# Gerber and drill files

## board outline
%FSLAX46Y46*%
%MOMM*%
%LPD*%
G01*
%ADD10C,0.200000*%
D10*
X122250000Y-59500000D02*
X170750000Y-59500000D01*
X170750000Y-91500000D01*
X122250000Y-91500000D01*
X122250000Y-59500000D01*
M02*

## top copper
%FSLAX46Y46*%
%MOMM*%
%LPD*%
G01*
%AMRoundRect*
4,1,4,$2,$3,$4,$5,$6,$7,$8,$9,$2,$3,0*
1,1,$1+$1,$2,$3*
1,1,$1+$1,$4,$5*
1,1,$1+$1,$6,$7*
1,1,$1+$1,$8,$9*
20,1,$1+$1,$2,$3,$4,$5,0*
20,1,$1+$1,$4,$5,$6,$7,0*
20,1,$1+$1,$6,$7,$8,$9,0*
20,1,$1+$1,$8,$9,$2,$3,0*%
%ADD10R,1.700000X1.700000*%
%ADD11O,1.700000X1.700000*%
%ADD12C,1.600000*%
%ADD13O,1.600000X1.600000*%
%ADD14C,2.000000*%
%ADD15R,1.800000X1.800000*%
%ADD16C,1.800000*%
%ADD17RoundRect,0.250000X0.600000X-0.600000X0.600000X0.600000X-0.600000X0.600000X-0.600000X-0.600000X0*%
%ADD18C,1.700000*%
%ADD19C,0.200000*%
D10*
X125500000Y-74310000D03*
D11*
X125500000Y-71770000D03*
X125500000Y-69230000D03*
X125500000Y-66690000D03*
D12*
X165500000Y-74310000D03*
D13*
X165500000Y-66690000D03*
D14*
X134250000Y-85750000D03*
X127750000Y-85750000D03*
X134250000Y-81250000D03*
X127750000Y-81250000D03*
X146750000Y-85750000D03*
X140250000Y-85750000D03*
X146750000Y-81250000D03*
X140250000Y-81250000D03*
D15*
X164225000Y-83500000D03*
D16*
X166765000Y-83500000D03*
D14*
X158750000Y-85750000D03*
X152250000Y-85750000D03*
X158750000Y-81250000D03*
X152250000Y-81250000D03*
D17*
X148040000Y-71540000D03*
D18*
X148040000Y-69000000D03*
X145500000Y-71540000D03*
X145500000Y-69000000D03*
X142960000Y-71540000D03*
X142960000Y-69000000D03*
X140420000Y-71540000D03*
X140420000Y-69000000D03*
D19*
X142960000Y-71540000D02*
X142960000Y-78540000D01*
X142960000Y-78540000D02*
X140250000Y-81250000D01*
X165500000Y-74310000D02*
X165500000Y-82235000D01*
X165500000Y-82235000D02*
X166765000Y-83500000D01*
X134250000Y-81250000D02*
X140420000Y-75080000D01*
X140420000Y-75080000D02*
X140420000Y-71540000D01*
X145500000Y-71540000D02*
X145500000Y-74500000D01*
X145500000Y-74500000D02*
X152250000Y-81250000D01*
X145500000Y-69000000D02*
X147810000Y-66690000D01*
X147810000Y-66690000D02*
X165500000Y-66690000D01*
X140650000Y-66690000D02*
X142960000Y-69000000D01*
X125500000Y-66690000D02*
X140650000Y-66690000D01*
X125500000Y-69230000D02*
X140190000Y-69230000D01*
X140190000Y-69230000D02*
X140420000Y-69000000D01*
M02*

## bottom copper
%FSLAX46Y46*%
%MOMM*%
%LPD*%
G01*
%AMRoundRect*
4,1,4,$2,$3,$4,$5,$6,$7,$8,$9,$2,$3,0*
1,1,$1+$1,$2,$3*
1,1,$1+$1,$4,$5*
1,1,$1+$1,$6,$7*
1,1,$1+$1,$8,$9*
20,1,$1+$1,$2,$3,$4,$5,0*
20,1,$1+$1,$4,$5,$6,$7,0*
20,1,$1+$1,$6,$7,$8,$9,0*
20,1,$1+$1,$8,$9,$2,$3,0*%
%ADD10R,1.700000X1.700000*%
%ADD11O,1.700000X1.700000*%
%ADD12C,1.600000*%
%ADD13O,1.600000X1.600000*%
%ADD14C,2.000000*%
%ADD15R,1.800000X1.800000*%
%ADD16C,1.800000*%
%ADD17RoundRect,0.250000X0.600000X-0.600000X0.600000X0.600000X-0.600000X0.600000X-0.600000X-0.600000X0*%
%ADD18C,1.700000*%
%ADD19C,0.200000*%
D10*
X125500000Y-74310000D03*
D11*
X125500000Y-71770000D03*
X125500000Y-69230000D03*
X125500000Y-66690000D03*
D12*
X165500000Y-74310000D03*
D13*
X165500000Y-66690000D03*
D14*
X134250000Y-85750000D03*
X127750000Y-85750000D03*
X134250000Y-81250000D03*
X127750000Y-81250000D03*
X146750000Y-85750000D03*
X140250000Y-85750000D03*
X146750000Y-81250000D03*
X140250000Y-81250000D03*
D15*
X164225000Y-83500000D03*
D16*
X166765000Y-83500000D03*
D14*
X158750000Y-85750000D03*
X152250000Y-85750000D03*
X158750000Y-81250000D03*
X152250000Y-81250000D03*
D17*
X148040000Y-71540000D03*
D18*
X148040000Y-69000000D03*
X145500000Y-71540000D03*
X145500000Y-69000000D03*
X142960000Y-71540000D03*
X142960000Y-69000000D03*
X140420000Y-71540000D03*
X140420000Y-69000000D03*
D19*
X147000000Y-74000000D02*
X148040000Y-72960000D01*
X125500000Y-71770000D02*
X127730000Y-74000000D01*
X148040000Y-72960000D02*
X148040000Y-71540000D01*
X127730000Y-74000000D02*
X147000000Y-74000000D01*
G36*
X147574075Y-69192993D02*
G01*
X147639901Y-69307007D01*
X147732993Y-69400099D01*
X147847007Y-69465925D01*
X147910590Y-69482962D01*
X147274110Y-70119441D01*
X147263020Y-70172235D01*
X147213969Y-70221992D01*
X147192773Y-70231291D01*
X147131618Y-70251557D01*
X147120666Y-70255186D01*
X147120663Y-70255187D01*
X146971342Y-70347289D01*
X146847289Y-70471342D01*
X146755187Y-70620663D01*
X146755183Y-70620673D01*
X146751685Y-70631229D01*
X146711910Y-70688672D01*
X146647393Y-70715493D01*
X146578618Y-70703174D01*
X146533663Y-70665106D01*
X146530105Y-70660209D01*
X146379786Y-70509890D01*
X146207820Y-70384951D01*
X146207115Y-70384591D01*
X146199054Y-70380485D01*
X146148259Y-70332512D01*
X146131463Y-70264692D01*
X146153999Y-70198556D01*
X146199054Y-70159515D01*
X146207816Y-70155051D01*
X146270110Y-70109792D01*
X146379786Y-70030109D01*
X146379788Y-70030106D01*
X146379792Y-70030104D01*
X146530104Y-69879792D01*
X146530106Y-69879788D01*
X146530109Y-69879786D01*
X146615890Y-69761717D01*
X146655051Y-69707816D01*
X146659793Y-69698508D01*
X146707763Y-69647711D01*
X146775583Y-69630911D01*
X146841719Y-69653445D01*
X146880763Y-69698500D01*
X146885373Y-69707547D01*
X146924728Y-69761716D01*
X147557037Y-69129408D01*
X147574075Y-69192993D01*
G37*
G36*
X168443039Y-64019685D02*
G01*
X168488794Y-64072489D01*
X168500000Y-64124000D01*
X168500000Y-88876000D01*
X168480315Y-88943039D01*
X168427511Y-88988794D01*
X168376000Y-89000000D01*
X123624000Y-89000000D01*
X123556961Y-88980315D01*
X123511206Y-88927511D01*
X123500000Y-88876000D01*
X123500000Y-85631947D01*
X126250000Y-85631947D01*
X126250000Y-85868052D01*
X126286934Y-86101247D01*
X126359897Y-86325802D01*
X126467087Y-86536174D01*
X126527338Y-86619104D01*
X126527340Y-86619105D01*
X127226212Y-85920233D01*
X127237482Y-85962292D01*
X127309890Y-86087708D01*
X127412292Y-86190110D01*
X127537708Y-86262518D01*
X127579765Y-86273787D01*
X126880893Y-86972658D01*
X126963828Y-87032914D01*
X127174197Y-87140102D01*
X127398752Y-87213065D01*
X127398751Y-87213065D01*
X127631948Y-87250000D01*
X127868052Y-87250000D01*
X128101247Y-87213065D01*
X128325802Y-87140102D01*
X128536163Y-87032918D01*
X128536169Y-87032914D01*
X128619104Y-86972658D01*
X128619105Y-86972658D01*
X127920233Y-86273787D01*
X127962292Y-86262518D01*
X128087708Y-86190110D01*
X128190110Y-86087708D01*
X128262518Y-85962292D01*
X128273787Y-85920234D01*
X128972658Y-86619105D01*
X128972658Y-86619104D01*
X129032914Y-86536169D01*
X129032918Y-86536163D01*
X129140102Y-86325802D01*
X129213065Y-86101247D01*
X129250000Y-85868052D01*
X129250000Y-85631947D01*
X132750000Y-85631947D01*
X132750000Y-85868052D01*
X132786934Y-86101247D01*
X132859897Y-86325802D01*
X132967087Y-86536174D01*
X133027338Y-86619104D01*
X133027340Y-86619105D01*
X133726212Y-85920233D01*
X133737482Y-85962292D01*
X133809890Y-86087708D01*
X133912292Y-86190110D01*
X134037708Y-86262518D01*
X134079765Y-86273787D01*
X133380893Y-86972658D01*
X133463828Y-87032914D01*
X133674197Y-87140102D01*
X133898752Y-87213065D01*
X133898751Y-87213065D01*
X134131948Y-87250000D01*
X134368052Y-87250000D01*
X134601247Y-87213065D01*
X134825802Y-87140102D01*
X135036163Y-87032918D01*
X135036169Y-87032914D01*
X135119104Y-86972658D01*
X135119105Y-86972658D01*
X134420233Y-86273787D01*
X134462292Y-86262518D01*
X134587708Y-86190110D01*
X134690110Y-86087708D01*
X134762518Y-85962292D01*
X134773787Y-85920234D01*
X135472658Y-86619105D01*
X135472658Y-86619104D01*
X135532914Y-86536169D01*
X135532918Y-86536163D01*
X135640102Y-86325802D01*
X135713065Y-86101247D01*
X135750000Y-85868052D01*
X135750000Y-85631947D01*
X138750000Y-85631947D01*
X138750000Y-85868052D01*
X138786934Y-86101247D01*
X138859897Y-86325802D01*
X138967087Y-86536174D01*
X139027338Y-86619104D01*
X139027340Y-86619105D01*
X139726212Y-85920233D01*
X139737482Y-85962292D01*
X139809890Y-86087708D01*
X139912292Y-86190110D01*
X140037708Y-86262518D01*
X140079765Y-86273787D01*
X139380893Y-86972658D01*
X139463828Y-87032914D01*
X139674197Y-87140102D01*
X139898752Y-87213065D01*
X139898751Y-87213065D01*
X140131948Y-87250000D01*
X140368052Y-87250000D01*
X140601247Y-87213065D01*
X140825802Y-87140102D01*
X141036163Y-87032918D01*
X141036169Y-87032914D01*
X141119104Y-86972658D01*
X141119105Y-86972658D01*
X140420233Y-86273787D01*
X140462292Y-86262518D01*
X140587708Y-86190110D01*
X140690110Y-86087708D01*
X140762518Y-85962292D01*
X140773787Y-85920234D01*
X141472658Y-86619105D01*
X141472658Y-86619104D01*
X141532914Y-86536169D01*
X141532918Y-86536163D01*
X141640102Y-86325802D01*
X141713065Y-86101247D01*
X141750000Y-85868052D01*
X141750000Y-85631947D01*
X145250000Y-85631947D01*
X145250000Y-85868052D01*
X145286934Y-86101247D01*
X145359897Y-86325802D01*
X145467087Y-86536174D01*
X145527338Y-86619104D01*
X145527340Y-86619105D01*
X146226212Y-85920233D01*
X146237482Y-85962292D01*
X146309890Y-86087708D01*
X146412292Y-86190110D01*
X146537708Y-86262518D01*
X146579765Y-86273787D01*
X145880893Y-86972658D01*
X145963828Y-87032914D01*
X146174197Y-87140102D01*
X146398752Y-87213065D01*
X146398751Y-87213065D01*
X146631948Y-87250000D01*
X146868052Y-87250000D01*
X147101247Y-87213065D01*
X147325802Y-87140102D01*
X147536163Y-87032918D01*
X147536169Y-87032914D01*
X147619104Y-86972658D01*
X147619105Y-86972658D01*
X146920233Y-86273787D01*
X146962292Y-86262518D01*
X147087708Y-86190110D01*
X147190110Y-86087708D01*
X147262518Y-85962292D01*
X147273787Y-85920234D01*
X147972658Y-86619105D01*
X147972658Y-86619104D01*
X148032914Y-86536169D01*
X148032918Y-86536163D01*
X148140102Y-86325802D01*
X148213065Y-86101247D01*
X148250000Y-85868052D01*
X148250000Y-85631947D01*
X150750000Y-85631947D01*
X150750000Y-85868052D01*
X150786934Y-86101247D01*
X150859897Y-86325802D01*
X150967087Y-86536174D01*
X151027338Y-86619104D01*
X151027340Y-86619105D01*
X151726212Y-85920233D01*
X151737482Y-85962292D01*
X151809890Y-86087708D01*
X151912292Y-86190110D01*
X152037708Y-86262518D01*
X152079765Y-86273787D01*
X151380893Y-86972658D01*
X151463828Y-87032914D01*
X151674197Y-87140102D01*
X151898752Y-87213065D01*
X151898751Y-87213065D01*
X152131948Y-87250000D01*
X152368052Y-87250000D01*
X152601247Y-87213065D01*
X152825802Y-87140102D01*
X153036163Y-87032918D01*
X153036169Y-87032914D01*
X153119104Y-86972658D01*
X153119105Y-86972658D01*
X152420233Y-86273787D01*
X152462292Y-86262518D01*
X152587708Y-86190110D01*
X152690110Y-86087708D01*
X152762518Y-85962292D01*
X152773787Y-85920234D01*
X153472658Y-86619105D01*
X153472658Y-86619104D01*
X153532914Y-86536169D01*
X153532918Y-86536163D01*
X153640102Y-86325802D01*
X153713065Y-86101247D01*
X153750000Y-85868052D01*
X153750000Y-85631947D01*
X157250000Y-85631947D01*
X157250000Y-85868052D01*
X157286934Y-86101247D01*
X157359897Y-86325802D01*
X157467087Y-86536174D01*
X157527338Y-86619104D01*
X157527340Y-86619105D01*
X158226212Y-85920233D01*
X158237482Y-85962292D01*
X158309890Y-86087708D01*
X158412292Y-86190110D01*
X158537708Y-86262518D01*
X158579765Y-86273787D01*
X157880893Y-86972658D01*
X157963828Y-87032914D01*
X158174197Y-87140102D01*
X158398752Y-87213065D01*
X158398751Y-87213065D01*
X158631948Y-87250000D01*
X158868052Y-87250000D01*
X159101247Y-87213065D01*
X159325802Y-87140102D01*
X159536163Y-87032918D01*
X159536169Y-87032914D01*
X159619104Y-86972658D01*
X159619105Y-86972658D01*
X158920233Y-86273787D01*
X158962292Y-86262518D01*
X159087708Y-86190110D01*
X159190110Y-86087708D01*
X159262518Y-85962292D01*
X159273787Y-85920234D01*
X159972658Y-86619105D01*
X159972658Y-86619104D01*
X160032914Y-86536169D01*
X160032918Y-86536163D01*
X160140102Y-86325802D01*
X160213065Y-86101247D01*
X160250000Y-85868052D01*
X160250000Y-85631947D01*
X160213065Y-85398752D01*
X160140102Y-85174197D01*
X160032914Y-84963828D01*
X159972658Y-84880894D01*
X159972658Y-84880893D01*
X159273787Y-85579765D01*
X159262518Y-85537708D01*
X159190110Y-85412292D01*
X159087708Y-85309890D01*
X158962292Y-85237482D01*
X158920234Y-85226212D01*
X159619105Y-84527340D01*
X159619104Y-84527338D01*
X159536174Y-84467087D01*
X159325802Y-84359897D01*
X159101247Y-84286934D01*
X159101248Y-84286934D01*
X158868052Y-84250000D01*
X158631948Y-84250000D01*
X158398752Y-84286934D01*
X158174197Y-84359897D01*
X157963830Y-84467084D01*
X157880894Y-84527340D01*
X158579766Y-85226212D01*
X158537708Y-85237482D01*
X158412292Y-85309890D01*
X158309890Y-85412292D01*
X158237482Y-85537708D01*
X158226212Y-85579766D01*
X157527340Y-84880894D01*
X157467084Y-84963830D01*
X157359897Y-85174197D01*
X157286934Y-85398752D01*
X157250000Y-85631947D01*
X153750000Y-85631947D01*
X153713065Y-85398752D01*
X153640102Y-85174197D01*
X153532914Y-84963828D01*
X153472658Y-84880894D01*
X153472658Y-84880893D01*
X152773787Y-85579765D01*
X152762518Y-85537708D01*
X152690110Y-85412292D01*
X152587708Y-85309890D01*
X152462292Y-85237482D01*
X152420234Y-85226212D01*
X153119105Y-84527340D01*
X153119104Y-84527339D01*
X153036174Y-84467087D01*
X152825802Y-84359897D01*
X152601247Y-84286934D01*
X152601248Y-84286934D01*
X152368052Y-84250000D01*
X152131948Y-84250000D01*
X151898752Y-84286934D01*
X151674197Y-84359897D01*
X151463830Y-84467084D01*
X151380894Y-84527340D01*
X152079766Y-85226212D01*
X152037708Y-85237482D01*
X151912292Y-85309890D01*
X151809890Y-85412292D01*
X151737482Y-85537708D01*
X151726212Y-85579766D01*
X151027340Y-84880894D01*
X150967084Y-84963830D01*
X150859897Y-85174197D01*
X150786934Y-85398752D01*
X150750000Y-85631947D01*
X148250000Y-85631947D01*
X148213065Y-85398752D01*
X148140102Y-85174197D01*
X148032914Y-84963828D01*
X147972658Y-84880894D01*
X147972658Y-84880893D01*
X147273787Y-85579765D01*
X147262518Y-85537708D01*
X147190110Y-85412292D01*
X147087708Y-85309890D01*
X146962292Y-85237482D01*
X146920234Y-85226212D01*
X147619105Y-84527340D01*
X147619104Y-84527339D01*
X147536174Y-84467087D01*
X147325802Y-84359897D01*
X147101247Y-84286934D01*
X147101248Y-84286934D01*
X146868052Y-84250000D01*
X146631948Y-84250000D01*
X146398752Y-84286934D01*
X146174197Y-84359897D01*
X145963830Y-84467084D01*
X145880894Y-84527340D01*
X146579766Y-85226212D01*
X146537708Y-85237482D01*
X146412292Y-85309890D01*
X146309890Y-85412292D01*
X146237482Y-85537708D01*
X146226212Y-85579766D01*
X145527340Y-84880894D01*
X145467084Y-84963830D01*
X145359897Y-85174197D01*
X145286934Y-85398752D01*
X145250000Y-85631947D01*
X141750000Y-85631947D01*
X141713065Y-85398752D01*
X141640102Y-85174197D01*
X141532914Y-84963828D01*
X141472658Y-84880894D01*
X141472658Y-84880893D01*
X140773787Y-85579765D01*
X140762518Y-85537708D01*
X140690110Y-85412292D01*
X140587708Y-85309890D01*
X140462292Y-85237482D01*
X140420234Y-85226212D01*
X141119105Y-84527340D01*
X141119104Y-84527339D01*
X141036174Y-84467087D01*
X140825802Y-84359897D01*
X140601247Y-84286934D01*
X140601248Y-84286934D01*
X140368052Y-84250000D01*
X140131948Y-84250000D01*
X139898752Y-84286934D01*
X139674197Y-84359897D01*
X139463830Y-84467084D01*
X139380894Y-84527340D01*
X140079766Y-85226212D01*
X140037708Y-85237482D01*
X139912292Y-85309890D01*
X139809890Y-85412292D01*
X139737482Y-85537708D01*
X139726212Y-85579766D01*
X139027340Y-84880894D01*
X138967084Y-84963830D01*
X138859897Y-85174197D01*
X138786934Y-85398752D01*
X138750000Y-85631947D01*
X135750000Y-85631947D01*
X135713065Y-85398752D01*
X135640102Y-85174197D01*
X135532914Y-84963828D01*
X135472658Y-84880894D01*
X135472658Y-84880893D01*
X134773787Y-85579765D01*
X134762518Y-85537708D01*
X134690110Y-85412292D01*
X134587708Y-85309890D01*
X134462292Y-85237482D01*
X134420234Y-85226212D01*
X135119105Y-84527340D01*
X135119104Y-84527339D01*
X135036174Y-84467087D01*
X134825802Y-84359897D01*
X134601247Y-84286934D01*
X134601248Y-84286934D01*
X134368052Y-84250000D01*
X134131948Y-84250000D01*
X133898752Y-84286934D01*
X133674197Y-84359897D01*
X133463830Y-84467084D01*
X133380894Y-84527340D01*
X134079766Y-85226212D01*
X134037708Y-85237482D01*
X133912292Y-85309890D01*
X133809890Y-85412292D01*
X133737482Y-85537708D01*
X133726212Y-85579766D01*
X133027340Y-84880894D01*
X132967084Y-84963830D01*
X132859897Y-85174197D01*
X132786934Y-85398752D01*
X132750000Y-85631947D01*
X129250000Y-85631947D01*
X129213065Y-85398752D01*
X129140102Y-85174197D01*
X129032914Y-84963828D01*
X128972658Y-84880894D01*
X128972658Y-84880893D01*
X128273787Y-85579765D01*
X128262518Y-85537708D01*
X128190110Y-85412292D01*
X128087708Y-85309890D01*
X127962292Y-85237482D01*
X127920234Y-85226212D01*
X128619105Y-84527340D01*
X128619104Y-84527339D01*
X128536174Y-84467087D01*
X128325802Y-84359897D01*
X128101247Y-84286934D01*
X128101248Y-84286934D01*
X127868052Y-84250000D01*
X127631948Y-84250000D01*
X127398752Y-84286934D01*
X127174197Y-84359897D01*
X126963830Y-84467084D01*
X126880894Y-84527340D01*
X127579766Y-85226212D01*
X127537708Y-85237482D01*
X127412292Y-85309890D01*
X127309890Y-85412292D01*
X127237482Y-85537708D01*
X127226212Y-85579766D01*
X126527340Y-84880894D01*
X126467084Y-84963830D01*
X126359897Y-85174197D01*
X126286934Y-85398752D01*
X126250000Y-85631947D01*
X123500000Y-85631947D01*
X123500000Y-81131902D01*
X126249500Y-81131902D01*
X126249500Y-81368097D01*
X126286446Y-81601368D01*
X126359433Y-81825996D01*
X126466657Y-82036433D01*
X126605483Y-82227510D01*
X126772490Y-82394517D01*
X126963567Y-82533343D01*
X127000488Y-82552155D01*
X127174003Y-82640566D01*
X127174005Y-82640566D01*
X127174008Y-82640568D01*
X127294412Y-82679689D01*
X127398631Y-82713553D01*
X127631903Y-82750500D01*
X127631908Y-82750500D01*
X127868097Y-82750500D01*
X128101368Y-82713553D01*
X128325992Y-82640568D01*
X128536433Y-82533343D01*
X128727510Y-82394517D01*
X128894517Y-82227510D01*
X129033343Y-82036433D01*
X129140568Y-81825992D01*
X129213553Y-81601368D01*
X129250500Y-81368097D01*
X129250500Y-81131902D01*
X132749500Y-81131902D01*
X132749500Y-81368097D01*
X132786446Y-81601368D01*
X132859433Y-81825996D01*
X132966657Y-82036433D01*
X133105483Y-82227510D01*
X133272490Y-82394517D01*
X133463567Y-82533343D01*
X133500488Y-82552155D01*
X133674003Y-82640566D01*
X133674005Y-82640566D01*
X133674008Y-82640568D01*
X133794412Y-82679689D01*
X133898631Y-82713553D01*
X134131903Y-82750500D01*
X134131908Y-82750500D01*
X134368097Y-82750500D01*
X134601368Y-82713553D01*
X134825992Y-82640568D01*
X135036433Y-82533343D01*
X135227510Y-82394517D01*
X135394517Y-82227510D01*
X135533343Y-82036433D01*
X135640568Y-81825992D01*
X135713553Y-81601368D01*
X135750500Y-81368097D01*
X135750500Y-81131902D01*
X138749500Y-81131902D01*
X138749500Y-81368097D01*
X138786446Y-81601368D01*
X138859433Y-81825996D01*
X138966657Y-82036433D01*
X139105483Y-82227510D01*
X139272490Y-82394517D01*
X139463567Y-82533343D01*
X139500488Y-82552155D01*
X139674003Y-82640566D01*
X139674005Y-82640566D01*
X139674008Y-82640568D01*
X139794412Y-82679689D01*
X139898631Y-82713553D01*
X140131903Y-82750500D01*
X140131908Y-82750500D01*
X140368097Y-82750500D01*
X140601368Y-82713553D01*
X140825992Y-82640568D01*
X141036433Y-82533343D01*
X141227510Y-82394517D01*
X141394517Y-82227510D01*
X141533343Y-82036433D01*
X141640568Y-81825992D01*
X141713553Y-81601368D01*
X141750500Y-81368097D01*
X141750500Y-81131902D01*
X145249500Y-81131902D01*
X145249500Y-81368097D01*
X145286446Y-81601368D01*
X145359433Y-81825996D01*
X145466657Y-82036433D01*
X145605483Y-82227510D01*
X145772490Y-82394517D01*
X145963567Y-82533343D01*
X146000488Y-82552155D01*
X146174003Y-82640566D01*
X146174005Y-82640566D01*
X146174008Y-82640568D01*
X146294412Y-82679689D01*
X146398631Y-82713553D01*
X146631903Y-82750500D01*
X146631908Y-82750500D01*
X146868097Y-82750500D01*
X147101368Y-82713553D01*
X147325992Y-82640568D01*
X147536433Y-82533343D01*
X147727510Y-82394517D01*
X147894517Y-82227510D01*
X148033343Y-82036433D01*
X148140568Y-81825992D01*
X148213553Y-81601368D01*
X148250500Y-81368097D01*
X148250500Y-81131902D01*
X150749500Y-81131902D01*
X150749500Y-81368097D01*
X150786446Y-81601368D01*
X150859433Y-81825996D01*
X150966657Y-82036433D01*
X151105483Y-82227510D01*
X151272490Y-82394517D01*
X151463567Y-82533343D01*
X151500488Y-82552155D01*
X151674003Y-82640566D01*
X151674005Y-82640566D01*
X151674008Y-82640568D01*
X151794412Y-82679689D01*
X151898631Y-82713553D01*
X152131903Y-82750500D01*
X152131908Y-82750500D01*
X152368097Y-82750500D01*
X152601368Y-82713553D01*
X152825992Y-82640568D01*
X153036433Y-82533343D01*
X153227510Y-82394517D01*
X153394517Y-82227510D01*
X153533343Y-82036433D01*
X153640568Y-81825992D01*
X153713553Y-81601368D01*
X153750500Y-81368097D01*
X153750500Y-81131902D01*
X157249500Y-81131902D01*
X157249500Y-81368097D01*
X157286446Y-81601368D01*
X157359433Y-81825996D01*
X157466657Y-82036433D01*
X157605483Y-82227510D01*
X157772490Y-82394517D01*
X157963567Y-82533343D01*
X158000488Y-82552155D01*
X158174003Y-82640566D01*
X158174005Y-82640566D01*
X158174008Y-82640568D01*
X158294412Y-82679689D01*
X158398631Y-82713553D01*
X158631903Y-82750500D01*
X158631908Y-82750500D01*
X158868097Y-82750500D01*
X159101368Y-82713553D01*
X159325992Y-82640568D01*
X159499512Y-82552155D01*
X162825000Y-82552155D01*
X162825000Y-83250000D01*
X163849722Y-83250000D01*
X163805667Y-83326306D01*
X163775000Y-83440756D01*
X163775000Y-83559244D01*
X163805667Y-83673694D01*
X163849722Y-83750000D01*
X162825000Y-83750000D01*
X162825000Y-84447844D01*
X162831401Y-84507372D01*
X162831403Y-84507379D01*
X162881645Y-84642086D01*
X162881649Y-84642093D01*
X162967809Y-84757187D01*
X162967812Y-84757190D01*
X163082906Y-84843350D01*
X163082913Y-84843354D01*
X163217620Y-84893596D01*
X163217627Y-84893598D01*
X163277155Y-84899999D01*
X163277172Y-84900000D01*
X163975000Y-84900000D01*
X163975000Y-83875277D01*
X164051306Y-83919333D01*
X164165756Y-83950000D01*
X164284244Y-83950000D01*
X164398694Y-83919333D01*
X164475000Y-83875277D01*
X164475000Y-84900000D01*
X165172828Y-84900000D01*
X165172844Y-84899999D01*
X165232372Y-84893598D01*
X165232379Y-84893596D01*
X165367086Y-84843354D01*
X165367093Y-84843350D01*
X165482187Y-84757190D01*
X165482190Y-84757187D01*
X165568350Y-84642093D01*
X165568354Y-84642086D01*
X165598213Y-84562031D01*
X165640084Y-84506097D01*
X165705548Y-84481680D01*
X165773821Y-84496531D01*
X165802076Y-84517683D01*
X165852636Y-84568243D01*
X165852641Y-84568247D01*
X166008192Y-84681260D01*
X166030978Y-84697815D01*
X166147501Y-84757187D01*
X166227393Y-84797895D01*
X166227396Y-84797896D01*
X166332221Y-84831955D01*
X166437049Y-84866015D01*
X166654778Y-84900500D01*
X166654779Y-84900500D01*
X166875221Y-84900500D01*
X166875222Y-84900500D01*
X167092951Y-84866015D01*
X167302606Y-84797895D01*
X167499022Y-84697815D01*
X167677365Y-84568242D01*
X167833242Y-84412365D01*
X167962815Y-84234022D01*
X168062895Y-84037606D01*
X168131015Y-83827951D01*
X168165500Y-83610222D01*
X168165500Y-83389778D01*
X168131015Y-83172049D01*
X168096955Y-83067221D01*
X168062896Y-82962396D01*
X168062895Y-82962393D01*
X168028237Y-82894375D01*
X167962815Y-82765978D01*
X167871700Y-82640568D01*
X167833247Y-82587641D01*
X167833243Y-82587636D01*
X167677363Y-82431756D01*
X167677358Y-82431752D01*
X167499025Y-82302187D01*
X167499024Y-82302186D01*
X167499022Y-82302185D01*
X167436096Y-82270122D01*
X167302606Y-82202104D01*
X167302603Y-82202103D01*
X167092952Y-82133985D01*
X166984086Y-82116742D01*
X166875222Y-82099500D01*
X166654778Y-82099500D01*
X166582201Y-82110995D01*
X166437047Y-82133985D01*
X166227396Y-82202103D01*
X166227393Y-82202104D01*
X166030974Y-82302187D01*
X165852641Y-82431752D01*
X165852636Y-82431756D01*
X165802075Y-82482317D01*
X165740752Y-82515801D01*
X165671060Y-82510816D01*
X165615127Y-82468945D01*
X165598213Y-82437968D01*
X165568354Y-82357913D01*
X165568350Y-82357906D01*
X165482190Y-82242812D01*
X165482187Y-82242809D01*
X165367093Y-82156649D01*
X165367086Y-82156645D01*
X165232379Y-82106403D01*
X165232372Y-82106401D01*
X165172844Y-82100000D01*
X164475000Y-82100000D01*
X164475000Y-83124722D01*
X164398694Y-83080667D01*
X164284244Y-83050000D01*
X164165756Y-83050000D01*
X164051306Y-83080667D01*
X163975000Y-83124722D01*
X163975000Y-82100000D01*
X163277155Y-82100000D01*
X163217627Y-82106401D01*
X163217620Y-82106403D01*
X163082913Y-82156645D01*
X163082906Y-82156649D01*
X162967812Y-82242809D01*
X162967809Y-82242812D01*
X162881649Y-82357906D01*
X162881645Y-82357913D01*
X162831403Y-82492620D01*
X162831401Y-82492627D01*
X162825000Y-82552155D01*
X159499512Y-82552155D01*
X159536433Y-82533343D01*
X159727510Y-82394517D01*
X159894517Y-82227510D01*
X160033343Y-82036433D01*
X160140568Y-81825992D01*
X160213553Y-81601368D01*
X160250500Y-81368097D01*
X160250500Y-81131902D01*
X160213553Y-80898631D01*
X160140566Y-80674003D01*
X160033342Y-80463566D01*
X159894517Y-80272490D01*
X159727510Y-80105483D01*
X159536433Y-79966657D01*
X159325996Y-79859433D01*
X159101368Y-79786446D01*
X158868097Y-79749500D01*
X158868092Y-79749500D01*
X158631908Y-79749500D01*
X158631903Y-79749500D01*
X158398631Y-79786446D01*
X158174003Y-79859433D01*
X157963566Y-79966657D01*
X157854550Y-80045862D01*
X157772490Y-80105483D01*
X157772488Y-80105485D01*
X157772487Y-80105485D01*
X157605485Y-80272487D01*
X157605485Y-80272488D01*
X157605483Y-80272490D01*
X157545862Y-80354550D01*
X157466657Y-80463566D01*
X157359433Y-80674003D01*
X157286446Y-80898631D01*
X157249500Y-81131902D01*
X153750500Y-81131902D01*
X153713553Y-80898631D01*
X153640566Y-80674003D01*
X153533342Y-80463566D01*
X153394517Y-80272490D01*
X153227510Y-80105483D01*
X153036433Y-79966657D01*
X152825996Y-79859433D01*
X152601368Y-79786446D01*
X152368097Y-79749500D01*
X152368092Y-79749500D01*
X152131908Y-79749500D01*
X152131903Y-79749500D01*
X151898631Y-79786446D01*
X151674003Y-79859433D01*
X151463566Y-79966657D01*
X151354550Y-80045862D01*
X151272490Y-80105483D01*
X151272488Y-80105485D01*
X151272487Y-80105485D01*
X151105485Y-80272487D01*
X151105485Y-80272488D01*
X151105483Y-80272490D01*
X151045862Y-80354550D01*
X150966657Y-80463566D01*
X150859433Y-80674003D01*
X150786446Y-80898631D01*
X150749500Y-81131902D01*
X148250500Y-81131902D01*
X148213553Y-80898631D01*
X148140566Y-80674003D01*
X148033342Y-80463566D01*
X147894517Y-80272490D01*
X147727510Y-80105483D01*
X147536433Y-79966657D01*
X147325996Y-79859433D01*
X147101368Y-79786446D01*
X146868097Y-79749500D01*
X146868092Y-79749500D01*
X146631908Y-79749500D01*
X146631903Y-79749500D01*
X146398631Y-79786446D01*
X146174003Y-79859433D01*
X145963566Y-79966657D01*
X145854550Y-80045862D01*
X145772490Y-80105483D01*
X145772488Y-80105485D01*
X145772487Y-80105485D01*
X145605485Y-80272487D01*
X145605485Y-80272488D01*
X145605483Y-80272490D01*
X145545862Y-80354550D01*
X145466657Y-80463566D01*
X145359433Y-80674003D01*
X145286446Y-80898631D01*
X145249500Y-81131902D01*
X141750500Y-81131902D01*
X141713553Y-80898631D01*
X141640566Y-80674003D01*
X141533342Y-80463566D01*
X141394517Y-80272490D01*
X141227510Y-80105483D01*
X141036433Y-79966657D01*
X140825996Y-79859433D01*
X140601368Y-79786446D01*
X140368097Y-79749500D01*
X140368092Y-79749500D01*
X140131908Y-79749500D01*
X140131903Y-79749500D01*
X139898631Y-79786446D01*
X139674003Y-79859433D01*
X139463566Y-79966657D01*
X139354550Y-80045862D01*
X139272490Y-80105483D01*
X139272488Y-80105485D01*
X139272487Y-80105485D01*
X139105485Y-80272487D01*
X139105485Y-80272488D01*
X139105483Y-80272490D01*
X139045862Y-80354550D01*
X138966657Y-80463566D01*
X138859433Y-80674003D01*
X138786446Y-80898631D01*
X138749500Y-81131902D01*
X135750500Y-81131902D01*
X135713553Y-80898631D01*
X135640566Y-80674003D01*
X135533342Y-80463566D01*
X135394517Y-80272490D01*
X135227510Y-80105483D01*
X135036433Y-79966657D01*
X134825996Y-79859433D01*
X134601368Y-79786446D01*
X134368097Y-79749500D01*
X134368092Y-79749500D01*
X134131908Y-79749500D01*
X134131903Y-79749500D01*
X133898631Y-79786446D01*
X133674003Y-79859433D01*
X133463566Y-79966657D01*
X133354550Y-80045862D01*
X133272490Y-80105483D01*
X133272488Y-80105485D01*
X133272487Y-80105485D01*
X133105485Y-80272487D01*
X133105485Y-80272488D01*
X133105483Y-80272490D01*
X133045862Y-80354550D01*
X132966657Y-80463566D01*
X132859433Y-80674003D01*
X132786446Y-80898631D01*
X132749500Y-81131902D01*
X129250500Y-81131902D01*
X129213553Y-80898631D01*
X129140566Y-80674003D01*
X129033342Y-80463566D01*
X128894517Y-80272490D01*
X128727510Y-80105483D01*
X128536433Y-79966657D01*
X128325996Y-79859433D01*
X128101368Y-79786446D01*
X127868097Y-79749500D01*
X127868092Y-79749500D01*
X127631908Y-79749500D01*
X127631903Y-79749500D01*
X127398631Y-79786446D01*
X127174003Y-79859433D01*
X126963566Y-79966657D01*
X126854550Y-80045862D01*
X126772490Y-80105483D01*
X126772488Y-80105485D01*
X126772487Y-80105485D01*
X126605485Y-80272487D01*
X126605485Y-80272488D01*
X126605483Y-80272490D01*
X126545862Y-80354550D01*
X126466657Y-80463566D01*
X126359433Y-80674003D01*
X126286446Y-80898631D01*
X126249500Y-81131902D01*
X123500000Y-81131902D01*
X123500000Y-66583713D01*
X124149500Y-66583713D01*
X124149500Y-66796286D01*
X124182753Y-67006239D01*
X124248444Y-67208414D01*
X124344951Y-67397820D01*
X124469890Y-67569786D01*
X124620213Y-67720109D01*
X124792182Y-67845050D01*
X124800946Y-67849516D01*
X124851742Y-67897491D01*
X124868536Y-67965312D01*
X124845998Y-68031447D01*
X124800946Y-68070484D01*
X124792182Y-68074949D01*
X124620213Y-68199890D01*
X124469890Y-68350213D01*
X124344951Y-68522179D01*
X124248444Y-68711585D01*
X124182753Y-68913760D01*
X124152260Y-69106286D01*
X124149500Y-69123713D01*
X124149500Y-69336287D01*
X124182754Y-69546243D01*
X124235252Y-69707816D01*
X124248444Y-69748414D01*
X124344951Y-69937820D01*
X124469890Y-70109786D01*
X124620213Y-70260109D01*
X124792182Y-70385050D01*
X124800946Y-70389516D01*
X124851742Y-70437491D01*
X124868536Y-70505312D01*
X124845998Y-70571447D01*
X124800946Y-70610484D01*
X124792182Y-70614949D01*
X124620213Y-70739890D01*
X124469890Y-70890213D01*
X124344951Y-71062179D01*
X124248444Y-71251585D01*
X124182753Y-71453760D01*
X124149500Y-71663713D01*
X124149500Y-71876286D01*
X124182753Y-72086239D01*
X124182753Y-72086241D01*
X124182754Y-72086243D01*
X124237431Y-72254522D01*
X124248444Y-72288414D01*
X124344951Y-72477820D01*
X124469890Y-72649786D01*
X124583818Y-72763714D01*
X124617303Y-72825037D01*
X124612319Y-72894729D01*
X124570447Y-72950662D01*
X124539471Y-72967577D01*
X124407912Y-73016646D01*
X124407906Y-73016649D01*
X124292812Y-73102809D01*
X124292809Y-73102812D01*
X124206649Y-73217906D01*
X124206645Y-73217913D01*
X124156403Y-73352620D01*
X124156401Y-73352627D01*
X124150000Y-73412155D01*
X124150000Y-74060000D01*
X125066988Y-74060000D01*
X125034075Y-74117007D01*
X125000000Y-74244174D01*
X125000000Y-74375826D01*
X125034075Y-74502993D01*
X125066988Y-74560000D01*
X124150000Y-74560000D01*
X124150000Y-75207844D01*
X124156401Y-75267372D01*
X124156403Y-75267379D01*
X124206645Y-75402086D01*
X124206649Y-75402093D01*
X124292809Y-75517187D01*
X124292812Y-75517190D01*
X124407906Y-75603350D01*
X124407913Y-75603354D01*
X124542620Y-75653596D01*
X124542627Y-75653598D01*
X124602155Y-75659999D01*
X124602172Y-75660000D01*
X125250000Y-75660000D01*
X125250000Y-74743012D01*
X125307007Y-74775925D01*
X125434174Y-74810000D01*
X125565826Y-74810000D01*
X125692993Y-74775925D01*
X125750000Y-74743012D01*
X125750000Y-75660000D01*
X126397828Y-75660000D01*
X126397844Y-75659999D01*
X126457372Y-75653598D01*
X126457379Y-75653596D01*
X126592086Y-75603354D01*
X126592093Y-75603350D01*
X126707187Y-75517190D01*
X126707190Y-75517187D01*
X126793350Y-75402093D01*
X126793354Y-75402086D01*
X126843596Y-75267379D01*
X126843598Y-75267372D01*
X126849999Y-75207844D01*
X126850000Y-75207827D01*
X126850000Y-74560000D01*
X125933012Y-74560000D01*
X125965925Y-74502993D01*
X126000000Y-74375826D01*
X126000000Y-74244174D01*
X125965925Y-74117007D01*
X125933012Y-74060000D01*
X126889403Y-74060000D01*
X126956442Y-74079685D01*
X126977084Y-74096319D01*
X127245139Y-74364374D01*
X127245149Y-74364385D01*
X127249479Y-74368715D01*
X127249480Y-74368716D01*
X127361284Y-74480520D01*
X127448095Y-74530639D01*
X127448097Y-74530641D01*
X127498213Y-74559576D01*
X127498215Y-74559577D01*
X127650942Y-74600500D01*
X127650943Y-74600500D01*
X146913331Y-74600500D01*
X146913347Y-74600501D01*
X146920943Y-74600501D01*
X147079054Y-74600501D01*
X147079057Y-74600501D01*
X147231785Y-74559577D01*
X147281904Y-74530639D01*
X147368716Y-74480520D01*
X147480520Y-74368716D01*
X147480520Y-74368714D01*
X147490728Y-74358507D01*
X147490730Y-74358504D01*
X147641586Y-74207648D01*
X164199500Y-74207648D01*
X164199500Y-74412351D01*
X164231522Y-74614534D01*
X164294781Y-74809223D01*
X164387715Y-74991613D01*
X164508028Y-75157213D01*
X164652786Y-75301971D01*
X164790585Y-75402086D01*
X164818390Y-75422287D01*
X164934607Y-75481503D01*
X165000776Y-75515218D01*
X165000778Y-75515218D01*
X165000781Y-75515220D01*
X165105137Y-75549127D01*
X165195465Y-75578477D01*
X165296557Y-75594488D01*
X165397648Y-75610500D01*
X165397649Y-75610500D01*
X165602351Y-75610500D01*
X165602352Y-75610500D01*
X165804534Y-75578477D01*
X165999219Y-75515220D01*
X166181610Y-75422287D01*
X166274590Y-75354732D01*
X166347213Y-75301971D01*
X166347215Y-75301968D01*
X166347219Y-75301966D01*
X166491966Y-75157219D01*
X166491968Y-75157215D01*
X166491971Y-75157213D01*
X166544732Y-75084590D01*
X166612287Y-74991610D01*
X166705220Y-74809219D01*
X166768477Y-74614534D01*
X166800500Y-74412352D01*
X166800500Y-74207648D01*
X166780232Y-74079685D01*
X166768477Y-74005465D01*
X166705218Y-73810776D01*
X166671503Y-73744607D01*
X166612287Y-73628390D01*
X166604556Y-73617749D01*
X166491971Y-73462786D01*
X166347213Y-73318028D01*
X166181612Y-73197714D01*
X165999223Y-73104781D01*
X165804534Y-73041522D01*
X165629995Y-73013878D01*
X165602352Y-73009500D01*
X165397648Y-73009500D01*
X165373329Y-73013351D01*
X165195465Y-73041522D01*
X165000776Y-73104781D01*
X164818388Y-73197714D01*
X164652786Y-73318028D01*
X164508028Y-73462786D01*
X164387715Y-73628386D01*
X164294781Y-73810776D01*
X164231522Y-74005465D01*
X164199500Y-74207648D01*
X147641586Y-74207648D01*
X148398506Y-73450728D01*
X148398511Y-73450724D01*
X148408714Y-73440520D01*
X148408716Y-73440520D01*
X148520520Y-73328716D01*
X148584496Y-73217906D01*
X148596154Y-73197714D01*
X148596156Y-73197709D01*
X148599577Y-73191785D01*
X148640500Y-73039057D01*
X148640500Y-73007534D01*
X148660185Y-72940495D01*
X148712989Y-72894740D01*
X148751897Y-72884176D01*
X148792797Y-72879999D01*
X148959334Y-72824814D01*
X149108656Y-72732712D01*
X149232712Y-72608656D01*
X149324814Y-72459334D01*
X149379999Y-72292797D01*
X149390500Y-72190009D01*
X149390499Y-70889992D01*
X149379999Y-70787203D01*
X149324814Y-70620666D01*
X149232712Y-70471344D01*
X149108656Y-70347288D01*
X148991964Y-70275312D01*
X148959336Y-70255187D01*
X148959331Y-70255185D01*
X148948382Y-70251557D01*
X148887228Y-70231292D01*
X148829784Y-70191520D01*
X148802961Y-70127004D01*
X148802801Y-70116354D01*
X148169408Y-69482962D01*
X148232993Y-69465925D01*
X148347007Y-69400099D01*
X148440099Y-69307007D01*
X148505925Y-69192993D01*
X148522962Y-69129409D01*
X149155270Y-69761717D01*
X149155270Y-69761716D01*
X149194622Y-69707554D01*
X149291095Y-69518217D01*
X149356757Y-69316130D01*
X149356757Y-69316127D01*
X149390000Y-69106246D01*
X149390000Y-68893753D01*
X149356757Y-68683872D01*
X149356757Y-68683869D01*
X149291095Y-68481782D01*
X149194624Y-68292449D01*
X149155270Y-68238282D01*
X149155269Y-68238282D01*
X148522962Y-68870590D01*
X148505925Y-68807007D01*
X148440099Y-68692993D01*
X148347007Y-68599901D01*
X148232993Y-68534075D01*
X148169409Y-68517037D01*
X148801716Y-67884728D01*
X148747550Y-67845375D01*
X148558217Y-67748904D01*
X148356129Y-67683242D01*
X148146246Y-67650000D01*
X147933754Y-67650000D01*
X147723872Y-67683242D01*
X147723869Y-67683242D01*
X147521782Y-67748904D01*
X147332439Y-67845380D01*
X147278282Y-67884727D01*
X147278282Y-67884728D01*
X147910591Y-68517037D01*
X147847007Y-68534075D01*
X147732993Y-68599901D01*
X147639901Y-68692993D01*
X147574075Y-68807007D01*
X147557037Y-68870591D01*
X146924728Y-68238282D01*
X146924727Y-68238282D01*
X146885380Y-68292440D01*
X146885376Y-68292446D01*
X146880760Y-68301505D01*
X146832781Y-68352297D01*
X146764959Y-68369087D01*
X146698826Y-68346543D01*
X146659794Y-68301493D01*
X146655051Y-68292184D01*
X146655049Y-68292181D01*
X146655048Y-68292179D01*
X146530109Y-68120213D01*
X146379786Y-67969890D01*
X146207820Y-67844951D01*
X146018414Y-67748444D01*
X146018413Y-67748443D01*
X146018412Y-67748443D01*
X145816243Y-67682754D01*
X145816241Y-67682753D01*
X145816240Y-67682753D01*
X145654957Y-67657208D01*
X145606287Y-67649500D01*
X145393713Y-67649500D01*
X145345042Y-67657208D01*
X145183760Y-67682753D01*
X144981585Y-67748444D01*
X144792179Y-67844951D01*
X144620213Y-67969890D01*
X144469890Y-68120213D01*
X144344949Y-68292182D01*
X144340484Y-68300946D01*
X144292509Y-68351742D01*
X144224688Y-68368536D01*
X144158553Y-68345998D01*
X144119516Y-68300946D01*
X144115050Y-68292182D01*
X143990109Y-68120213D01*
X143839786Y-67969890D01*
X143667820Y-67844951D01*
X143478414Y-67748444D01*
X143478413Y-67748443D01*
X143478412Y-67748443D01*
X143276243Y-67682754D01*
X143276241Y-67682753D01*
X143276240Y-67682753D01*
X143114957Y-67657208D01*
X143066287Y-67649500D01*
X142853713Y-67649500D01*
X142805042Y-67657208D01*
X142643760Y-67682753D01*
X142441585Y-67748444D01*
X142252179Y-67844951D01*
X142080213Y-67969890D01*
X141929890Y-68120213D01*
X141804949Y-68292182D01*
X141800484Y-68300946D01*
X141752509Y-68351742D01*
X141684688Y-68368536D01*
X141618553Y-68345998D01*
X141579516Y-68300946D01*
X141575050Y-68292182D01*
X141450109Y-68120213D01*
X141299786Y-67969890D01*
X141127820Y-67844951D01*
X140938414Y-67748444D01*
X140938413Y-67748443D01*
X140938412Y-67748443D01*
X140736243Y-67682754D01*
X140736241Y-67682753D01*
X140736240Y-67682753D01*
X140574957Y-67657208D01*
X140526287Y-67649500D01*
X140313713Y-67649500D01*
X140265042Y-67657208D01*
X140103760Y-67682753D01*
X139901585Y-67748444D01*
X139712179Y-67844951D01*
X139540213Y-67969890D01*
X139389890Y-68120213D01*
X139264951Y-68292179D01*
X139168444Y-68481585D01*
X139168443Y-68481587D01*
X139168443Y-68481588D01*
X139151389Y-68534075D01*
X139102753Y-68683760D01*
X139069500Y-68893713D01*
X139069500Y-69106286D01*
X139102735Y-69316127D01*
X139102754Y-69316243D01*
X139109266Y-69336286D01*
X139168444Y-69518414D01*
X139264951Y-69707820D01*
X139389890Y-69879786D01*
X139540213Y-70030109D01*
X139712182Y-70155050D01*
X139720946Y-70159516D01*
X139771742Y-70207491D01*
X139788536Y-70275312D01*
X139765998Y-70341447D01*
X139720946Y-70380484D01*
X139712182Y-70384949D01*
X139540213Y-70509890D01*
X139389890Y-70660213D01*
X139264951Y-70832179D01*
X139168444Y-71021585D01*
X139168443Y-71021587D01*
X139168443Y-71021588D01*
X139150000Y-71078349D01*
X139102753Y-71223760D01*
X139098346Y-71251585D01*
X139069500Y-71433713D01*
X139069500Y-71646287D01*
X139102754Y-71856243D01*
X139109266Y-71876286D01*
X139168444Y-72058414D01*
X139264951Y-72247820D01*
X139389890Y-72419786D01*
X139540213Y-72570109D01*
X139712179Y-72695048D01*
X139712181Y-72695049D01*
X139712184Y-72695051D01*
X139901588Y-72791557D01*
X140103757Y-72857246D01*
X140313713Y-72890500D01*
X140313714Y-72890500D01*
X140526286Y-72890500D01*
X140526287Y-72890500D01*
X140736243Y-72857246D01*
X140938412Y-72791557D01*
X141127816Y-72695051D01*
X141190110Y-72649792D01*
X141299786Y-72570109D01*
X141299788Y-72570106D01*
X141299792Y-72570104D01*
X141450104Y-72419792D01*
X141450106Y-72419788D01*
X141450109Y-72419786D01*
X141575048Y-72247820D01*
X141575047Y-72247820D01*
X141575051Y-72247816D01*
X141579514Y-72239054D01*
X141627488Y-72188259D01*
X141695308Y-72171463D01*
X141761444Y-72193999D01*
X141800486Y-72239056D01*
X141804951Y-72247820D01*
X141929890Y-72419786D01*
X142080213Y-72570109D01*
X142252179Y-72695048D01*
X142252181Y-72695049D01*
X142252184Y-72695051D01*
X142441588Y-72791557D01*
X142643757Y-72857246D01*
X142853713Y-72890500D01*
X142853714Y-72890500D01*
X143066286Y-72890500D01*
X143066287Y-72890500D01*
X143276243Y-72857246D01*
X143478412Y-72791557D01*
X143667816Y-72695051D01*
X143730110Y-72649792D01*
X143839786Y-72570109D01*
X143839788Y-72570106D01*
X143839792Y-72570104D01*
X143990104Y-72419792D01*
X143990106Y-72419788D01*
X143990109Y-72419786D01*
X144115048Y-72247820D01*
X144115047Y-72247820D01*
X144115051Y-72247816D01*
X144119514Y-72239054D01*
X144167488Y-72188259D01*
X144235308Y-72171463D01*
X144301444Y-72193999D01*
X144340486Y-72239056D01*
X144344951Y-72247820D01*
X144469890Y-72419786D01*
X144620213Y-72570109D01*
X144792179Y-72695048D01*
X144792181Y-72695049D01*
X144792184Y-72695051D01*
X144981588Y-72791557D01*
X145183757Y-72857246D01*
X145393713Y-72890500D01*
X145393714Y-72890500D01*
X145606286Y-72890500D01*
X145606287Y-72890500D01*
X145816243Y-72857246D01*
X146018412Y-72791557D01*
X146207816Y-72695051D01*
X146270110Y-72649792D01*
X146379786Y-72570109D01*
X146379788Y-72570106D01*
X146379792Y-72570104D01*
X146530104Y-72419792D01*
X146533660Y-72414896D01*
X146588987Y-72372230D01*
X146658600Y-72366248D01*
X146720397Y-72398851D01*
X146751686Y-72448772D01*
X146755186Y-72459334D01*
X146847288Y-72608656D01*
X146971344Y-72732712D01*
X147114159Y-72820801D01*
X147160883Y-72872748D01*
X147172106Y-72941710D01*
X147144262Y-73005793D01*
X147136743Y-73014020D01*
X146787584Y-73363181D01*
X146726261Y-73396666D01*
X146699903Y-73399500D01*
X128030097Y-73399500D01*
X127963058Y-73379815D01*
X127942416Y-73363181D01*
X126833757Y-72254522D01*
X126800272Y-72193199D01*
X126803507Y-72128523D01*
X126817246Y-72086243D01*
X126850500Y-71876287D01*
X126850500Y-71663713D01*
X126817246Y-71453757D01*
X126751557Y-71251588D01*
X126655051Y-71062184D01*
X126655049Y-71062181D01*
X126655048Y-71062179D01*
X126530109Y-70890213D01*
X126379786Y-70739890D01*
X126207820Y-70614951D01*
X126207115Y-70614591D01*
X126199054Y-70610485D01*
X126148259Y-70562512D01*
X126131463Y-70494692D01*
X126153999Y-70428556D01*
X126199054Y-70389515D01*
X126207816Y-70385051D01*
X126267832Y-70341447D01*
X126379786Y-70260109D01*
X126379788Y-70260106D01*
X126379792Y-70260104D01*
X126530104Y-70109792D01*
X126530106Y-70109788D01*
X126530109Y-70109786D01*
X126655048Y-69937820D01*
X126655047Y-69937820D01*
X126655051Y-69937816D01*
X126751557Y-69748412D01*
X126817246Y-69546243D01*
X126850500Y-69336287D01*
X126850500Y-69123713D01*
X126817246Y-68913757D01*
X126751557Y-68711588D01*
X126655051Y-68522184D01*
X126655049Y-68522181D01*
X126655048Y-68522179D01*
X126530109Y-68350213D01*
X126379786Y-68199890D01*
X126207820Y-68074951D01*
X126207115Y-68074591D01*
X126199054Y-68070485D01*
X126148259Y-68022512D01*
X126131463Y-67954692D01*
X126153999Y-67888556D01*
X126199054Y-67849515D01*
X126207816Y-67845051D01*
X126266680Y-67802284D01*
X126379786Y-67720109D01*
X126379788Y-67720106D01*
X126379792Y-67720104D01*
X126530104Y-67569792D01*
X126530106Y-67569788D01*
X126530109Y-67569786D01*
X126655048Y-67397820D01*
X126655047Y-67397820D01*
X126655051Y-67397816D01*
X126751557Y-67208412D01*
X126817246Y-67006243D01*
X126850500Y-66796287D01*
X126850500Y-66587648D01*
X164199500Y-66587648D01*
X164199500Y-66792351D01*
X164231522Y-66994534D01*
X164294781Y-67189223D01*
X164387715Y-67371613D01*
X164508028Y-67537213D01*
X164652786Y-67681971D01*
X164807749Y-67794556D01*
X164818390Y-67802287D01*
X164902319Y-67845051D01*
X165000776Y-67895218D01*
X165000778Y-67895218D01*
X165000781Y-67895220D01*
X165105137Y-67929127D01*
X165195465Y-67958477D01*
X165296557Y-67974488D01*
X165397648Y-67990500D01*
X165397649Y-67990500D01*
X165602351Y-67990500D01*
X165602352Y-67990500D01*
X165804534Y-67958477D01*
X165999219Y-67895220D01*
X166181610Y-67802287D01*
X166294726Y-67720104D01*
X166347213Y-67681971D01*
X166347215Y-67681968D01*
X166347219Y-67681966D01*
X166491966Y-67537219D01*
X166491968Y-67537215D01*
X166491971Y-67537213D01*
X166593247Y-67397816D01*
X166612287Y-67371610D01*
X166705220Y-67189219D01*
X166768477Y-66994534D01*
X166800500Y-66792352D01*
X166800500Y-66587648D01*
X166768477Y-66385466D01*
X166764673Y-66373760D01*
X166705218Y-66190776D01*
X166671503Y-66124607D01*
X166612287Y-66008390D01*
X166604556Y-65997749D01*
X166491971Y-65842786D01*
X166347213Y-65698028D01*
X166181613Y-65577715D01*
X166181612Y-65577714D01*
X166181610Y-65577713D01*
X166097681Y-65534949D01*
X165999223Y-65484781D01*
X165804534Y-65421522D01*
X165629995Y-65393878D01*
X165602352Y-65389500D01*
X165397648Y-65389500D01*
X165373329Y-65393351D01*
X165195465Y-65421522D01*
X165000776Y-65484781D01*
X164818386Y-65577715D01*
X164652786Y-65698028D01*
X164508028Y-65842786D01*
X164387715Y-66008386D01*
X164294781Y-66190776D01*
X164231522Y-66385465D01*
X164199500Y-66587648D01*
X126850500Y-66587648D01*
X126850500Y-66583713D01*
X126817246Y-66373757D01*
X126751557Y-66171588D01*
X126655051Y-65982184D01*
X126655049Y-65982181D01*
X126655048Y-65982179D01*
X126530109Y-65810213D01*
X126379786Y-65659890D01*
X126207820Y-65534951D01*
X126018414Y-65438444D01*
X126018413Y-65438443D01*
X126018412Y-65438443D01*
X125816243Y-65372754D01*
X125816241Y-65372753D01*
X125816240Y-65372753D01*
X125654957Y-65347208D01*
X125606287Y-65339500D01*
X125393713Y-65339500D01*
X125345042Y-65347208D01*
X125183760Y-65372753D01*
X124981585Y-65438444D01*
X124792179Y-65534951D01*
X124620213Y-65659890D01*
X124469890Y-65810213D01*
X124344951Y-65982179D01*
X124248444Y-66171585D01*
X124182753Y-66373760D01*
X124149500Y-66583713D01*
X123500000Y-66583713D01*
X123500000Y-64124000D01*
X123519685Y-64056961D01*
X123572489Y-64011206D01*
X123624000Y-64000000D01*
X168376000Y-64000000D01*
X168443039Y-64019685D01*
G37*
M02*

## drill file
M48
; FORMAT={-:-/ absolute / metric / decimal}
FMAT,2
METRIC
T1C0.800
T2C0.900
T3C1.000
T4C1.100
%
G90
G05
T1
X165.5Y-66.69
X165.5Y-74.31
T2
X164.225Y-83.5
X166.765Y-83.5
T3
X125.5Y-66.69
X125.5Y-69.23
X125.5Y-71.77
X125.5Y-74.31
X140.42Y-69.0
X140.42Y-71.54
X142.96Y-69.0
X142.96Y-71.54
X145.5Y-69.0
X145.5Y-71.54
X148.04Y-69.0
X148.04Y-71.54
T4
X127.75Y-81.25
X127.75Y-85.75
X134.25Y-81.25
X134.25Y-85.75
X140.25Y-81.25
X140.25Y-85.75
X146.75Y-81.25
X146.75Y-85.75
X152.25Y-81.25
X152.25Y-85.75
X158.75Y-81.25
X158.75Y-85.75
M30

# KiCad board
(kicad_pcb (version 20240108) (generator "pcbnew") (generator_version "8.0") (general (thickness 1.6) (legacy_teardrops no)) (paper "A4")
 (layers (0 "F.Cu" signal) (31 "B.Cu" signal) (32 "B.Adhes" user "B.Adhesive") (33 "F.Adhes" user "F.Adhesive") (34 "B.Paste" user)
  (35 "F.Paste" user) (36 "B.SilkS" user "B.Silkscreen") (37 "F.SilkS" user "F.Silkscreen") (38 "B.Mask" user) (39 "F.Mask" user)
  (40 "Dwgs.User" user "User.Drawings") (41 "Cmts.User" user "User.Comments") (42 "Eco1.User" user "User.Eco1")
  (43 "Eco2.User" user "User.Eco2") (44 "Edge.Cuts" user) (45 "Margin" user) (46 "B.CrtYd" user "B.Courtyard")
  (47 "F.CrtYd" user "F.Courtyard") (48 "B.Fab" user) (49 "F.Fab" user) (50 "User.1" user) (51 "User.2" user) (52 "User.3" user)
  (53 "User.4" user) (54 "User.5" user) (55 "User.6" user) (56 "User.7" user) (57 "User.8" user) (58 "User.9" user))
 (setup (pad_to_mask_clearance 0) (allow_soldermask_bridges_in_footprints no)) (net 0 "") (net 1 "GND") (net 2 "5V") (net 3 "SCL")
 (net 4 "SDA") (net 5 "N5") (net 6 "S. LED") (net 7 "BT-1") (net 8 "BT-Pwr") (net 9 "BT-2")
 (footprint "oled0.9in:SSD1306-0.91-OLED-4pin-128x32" (layer "F.Cu") (at 162 76.5 180)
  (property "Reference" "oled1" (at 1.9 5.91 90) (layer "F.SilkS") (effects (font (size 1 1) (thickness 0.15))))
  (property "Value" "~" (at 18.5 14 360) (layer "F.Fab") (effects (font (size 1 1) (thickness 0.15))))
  (pad "1" thru_hole rect (at 36.5 2.19 180) (size 1.7 1.7) (drill 1) (layers "*.Cu" "*.Mask") (remove_unused_layers no) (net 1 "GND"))
  (pad "2" thru_hole oval (at 36.5 4.73 180) (size 1.7 1.7) (drill 1) (layers "*.Cu" "*.Mask") (remove_unused_layers no) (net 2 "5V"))
  (pad "3" thru_hole oval (at 36.5 7.27 180) (size 1.7 1.7) (drill 1) (layers "*.Cu" "*.Mask") (remove_unused_layers no) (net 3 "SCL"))
  (pad "4" thru_hole oval (at 36.5 9.81 180) (size 1.7 1.7) (drill 1) (layers "*.Cu" "*.Mask") (remove_unused_layers no) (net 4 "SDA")))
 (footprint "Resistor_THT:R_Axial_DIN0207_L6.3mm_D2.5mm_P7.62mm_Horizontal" (layer "F.Cu") (at 165.5 74.31 90)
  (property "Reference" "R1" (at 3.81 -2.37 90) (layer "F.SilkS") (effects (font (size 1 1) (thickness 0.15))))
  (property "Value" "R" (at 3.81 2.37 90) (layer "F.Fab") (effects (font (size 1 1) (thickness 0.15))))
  (pad "1" thru_hole circle (at 0 0 90) (size 1.6 1.6) (drill 0.8) (layers "*.Cu" "*.Mask") (remove_unused_layers no) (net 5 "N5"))
  (pad "2" thru_hole oval (at 7.62 0 90) (size 1.6 1.6) (drill 0.8) (layers "*.Cu" "*.Mask") (remove_unused_layers no) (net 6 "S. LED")))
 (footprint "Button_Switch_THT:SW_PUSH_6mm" (layer "F.Cu") (at 134.25 85.75 180)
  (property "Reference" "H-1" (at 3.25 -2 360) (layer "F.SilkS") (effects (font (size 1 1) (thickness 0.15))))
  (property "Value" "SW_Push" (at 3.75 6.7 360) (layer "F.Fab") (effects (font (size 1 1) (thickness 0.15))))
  (pad "1" thru_hole circle (at 0 0 270) (size 2 2) (drill 1.1) (layers "*.Cu" "*.Mask") (remove_unused_layers no) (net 1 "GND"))
  (pad "1" thru_hole circle (at 6.5 0 270) (size 2 2) (drill 1.1) (layers "*.Cu" "*.Mask") (remove_unused_layers no) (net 1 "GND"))
  (pad "2" thru_hole circle (at 0 4.5 270) (size 2 2) (drill 1.1) (layers "*.Cu" "*.Mask") (remove_unused_layers no) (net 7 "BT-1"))
  (pad "2" thru_hole circle (at 6.5 4.5 270) (size 2 2) (drill 1.1) (layers "*.Cu" "*.Mask") (remove_unused_layers no) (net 7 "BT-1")))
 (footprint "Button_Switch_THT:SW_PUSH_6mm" (layer "F.Cu") (at 146.75 85.75 180)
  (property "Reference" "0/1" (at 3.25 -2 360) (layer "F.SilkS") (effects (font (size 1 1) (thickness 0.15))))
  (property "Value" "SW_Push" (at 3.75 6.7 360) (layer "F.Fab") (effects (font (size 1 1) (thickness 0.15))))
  (pad "1" thru_hole circle (at 0 0 270) (size 2 2) (drill 1.1) (layers "*.Cu" "*.Mask") (remove_unused_layers no) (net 1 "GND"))
  (pad "1" thru_hole circle (at 6.5 0 270) (size 2 2) (drill 1.1) (layers "*.Cu" "*.Mask") (remove_unused_layers no) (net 1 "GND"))
  (pad "2" thru_hole circle (at 0 4.5 270) (size 2 2) (drill 1.1) (layers "*.Cu" "*.Mask") (remove_unused_layers no) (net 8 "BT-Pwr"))
  (pad "2" thru_hole circle (at 6.5 4.5 270) (size 2 2) (drill 1.1) (layers "*.Cu" "*.Mask") (remove_unused_layers no) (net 8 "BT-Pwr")))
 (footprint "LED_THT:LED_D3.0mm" (layer "F.Cu") (at 164.225 83.5)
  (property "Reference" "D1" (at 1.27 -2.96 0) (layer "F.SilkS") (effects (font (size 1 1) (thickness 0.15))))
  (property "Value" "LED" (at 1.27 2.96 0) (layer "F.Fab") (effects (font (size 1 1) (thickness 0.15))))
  (pad "1" thru_hole rect (at 0 0) (size 1.8 1.8) (drill 0.9) (layers "*.Cu" "*.Mask") (remove_unused_layers no) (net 1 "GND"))
  (pad "2" thru_hole circle (at 2.54 0) (size 1.8 1.8) (drill 0.9) (layers "*.Cu" "*.Mask") (remove_unused_layers no) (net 5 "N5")))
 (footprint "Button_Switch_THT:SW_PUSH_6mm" (layer "F.Cu") (at 158.75 85.75 180)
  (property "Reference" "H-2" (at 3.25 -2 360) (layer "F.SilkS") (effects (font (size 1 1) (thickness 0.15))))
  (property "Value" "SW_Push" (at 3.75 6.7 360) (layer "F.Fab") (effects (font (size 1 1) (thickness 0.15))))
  (pad "1" thru_hole circle (at 0 0 270) (size 2 2) (drill 1.1) (layers "*.Cu" "*.Mask") (remove_unused_layers no) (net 1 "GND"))
  (pad "1" thru_hole circle (at 6.5 0 270) (size 2 2) (drill 1.1) (layers "*.Cu" "*.Mask") (remove_unused_layers no) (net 1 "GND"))
  (pad "2" thru_hole circle (at 0 4.5 270) (size 2 2) (drill 1.1) (layers "*.Cu" "*.Mask") (remove_unused_layers no) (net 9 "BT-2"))
  (pad "2" thru_hole circle (at 6.5 4.5 270) (size 2 2) (drill 1.1) (layers "*.Cu" "*.Mask") (remove_unused_layers no) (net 9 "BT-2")))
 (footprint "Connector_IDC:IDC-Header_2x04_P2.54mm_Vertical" (layer "B.Cu") (at 148.04 71.54 90)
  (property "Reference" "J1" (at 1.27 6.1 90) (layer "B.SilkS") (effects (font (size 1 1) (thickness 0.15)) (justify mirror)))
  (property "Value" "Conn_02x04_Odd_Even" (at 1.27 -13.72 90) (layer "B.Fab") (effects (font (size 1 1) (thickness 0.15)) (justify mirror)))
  (pad "1" thru_hole roundrect (at 0 0 90) (size 1.7 1.7) (drill 1) (layers "*.Cu" "*.Mask") (remove_unused_layers no)
   (roundrect_rratio 0.147059) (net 2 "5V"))
  (pad "2" thru_hole circle (at 2.54 0 90) (size 1.7 1.7) (drill 1) (layers "*.Cu" "*.Mask") (remove_unused_layers no) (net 1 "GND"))
  (pad "3" thru_hole circle (at 0 -2.54 90) (size 1.7 1.7) (drill 1) (layers "*.Cu" "*.Mask") (remove_unused_layers no) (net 9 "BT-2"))
  (pad "4" thru_hole circle (at 2.54 -2.54 90) (size 1.7 1.7) (drill 1) (layers "*.Cu" "*.Mask") (remove_unused_layers no) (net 6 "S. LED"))
  (pad "5" thru_hole circle (at 0 -5.08 90) (size 1.7 1.7) (drill 1) (layers "*.Cu" "*.Mask") (remove_unused_layers no) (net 8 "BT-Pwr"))
  (pad "6" thru_hole circle (at 2.54 -5.08 90) (size 1.7 1.7) (drill 1) (layers "*.Cu" "*.Mask") (remove_unused_layers no) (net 4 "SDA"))
  (pad "7" thru_hole circle (at 0 -7.62 90) (size 1.7 1.7) (drill 1) (layers "*.Cu" "*.Mask") (remove_unused_layers no) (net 7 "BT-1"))
  (pad "8" thru_hole circle (at 2.54 -7.62 90) (size 1.7 1.7) (drill 1) (layers "*.Cu" "*.Mask") (remove_unused_layers no) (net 3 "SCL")))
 (gr_rect (start 122.25 59.5) (end 170.75 91.5) (stroke (width 0.2) (type default)) (fill none) (layer "Edge.Cuts"))
 (segment (start 142.96 71.54) (end 142.96 78.54) (width 0.2) (layer "F.Cu") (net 8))
 (segment (start 142.96 78.54) (end 140.25 81.25) (width 0.2) (layer "F.Cu") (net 8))
 (segment (start 165.5 74.31) (end 165.5 82.235) (width 0.2) (layer "F.Cu") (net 5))
 (segment (start 165.5 82.235) (end 166.765 83.5) (width 0.2) (layer "F.Cu") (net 5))
 (segment (start 134.25 81.25) (end 140.42 75.08) (width 0.2) (layer "F.Cu") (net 7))
 (segment (start 140.42 75.08) (end 140.42 71.54) (width 0.2) (layer "F.Cu") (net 7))
 (segment (start 145.5 71.54) (end 145.5 74.5) (width 0.2) (layer "F.Cu") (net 9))
 (segment (start 145.5 74.5) (end 152.25 81.25) (width 0.2) (layer "F.Cu") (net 9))
 (segment (start 145.5 69) (end 147.81 66.69) (width 0.2) (layer "F.Cu") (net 6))
 (segment (start 147.81 66.69) (end 165.5 66.69) (width 0.2) (layer "F.Cu") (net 6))
 (segment (start 140.65 66.69) (end 142.96 69) (width 0.2) (layer "F.Cu") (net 4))
 (segment (start 125.5 66.69) (end 140.65 66.69) (width 0.2) (layer "F.Cu") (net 4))
 (segment (start 147 74) (end 148.04 72.96) (width 0.2) (layer "B.Cu") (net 2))
 (segment (start 125.5 71.77) (end 127.73 74) (width 0.2) (layer "B.Cu") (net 2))
 (segment (start 148.04 72.96) (end 148.04 71.54) (width 0.2) (layer "B.Cu") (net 2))
 (segment (start 127.73 74) (end 147 74) (width 0.2) (layer "B.Cu") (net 2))
 (segment (start 125.5 69.23) (end 140.19 69.23) (width 0.2) (layer "F.Cu") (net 3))
 (segment (start 140.19 69.23) (end 140.42 69) (width 0.2) (layer "F.Cu") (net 3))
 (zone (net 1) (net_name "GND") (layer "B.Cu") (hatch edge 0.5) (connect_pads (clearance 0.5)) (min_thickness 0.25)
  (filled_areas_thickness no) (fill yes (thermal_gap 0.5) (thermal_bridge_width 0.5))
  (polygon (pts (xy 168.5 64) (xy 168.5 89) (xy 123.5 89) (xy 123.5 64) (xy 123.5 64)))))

